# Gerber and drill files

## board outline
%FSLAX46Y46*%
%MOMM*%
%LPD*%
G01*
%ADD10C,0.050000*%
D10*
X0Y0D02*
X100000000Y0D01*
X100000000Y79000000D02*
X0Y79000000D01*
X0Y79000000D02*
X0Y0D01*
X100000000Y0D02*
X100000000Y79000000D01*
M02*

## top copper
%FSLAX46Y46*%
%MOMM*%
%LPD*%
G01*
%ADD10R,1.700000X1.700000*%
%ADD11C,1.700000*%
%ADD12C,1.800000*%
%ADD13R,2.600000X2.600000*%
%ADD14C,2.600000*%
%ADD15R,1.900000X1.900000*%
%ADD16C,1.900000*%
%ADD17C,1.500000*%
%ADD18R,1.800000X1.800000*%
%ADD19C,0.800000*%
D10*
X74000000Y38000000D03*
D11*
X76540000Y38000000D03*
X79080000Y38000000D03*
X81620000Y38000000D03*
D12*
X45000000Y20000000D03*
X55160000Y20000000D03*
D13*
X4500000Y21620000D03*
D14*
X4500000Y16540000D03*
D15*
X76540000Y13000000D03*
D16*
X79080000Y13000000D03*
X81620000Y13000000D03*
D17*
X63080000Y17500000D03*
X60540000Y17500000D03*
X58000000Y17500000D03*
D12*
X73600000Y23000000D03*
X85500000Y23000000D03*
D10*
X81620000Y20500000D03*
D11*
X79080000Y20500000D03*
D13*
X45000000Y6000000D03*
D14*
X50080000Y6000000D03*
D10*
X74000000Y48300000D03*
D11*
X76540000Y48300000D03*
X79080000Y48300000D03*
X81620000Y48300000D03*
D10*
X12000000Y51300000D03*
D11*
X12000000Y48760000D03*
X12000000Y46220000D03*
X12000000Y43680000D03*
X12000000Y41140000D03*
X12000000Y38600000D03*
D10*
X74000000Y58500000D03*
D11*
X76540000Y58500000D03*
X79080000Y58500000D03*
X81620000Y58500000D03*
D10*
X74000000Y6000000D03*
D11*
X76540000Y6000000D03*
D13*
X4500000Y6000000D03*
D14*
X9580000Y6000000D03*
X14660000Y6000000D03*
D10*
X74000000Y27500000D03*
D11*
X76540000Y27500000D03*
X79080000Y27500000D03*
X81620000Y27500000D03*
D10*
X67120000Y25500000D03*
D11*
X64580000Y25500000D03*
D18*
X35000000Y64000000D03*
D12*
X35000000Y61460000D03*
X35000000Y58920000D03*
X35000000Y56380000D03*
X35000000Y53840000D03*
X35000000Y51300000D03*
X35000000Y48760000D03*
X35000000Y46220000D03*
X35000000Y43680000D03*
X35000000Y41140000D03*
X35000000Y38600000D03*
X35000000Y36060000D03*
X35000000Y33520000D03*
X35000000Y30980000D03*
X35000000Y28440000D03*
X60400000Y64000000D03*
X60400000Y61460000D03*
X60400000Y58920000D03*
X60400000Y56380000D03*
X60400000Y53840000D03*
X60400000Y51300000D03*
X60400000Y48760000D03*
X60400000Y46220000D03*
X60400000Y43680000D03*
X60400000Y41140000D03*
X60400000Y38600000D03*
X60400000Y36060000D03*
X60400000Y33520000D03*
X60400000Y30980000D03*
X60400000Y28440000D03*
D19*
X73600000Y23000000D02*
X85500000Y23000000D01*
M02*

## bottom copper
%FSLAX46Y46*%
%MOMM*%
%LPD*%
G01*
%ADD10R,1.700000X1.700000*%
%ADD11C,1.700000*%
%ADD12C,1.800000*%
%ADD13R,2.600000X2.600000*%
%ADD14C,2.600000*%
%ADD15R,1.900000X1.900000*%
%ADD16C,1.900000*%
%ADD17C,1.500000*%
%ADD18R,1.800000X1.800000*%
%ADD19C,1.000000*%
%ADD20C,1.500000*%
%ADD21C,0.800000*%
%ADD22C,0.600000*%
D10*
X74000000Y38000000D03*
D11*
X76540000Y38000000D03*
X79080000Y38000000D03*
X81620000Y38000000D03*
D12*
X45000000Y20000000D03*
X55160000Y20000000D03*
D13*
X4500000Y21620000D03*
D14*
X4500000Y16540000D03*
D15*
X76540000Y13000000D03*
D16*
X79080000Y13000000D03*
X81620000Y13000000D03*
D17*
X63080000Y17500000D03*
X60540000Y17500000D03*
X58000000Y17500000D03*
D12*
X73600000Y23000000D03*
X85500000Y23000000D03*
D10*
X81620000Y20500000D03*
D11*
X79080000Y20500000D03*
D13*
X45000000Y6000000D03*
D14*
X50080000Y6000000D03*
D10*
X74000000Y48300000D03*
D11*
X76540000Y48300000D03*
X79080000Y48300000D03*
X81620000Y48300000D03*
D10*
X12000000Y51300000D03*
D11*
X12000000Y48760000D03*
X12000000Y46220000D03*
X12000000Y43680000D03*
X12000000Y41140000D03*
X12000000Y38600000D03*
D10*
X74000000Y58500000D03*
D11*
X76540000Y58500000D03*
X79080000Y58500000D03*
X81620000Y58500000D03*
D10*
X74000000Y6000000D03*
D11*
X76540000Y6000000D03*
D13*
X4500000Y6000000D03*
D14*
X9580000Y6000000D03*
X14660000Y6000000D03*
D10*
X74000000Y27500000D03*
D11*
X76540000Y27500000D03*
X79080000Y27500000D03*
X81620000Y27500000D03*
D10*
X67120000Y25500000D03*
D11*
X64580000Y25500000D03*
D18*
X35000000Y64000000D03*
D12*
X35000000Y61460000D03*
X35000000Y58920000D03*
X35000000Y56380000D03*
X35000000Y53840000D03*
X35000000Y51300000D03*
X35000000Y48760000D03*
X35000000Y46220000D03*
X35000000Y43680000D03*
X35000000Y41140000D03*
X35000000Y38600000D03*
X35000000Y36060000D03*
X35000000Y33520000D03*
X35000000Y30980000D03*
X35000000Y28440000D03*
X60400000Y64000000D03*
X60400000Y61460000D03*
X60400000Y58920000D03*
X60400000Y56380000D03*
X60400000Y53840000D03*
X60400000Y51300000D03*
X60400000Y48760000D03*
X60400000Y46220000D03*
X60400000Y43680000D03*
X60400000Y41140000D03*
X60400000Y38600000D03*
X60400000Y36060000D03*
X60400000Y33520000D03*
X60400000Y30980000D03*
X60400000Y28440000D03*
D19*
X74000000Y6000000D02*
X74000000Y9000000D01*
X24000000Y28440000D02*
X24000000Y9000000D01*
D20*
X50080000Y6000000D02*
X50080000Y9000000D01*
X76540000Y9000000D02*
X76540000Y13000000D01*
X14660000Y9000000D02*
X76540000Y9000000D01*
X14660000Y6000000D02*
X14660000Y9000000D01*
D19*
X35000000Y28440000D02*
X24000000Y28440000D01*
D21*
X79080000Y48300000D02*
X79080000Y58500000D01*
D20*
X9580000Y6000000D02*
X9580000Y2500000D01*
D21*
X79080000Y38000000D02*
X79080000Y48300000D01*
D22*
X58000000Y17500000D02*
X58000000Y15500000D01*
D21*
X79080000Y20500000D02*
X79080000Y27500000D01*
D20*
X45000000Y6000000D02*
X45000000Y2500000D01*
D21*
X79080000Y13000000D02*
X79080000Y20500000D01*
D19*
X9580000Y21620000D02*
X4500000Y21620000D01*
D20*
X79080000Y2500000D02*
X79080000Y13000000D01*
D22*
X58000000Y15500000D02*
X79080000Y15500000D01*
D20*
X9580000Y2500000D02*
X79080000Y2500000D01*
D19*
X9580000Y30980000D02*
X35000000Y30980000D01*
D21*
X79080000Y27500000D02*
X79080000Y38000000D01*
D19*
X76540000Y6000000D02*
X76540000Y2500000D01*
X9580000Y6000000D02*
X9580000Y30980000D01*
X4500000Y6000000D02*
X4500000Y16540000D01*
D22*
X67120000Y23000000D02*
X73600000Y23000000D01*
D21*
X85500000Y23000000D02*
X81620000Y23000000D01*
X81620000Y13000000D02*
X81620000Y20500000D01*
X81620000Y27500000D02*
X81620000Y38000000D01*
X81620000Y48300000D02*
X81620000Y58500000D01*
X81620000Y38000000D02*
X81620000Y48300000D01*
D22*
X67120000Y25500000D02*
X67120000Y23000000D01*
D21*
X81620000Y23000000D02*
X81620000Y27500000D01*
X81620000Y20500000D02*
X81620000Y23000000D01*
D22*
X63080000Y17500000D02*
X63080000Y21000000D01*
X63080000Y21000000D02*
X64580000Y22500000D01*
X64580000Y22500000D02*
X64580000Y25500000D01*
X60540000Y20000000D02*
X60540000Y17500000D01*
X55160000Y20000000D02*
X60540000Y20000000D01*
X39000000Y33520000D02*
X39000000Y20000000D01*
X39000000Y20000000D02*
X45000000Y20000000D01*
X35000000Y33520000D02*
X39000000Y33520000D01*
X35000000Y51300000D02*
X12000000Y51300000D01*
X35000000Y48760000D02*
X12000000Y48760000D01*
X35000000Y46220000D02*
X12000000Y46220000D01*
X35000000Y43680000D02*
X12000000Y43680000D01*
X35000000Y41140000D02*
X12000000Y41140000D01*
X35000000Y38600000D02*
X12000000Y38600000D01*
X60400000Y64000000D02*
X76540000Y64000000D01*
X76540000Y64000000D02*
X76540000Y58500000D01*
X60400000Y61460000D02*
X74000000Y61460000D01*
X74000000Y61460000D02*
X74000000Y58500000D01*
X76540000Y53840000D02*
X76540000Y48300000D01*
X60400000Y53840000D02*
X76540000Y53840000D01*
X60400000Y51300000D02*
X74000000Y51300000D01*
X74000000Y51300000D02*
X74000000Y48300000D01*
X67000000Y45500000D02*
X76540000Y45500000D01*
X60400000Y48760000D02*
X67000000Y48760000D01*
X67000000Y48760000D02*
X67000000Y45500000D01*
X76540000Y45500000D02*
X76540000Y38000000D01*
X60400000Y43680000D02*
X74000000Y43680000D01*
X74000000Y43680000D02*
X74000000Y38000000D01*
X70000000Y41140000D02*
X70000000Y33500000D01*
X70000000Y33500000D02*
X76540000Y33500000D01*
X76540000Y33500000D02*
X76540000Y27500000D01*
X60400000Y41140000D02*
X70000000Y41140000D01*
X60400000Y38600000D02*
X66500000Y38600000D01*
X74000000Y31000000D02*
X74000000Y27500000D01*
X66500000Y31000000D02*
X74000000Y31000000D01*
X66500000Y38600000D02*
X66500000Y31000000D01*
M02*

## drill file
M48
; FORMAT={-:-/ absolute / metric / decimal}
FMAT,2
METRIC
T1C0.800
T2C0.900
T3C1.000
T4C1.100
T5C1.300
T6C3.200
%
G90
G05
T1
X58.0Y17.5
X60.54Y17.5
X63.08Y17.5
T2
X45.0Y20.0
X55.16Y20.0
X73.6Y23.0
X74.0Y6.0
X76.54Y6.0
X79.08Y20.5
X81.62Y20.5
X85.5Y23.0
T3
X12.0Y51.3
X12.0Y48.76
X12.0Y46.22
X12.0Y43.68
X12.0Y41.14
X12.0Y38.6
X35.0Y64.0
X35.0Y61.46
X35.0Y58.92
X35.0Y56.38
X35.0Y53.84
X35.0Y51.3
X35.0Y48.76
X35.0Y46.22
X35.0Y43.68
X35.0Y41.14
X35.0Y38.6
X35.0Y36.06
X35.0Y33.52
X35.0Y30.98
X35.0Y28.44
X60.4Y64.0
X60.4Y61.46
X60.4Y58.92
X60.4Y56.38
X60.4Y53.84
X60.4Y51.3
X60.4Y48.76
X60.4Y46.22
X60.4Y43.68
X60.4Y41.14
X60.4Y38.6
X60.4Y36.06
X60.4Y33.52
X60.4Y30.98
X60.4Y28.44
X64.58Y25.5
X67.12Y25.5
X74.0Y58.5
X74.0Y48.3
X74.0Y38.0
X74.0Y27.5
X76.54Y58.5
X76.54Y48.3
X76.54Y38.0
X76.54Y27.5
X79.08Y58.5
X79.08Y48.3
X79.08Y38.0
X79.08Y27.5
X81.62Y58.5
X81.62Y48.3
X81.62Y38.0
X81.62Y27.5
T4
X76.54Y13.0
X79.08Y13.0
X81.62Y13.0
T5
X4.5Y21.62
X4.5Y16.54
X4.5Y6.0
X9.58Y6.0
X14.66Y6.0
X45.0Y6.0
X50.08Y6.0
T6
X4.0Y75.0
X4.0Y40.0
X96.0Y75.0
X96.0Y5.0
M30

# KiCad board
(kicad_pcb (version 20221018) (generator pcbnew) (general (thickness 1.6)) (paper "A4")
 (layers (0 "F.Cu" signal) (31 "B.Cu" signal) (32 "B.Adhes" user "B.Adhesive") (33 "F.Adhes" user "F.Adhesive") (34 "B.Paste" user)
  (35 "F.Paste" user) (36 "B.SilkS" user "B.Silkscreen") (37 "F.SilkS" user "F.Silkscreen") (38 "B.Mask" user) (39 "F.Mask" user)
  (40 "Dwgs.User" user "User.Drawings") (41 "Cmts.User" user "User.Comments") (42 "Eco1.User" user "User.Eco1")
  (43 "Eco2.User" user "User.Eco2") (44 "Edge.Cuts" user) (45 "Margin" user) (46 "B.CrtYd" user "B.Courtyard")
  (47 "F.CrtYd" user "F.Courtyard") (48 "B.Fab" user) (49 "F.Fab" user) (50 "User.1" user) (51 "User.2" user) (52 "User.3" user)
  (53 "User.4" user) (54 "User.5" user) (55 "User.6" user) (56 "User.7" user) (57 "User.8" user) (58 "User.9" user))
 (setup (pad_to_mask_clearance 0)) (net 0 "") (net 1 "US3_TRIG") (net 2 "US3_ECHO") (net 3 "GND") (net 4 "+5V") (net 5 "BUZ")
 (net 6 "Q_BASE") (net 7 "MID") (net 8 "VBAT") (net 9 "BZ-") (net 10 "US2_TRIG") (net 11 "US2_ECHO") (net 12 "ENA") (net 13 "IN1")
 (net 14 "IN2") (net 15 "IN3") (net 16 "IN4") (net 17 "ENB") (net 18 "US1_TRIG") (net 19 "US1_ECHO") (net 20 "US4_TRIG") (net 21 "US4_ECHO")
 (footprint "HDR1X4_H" (layer "F.Cu") (at 77.81 -38)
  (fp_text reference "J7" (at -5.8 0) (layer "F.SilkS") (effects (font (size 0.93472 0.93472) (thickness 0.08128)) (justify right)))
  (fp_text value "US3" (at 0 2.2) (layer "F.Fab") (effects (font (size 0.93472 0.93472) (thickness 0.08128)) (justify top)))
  (pad "1" thru_hole rect (at -3.81 0) (size 1.7 1.7) (drill 1) (layers "*.Cu" "*.Mask") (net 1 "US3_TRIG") (solder_mask_margin 0.1)
   (thermal_bridge_angle 0))
  (pad "2" thru_hole circle (at -1.27 0) (size 1.7 1.7) (drill 1) (layers "*.Cu" "*.Mask") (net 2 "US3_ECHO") (solder_mask_margin 0.1)
   (thermal_bridge_angle 0))
  (pad "3" thru_hole circle (at 1.27 0) (size 1.7 1.7) (drill 1) (layers "*.Cu" "*.Mask") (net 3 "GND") (solder_mask_margin 0.1)
   (thermal_bridge_angle 0))
  (pad "4" thru_hole circle (at 3.81 0) (size 1.7 1.7) (drill 1) (layers "*.Cu" "*.Mask") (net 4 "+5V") (solder_mask_margin 0.1)
   (thermal_bridge_angle 0)))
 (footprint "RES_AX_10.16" (layer "F.Cu") (at 50.08 -20)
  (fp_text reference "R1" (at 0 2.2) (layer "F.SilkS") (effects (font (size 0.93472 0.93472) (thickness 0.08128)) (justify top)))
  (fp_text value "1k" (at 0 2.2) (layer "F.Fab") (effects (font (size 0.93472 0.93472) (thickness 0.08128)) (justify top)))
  (pad "1" thru_hole circle (at -5.08 0) (size 1.8 1.8) (drill 0.9) (layers "*.Cu" "*.Mask") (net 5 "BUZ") (solder_mask_margin 0.1)
   (thermal_bridge_angle 0))
  (pad "2" thru_hole circle (at 5.08 0) (size 1.8 1.8) (drill 0.9) (layers "*.Cu" "*.Mask") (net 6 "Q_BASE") (solder_mask_margin 0.1)
   (thermal_bridge_angle 0)))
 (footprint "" (layer "F.Cu") (at 96 -75)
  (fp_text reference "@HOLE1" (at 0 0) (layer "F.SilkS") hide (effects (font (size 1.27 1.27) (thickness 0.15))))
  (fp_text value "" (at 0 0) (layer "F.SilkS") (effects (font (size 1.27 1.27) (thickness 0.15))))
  (pad "" np_thru_hole circle (at 0 0) (size 3.2 3.2) (drill 3.2) (layers "*.Cu" "*.Mask")))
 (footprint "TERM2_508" (layer "F.Cu") (at 4.5 -19.08 -90)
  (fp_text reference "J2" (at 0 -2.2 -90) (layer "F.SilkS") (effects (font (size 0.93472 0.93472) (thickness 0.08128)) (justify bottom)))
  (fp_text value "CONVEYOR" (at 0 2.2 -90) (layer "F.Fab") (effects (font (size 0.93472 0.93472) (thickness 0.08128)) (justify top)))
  (pad "1" thru_hole rect (at -2.54 0 270) (size 2.6 2.6) (drill 1.3) (layers "*.Cu" "*.Mask") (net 3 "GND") (solder_mask_margin 0.1)
   (thermal_bridge_angle 0))
  (pad "2" thru_hole circle (at 2.54 0 270) (size 2.6 2.6) (drill 1.3) (layers "*.Cu" "*.Mask") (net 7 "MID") (solder_mask_margin 0.1)
   (thermal_bridge_angle 0)))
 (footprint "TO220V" (layer "F.Cu") (at 79.08 -13)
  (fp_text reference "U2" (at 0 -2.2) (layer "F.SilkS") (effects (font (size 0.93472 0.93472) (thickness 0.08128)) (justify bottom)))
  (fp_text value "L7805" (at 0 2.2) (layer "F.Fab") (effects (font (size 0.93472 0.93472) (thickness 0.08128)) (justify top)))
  (pad "1" thru_hole rect (at -2.54 0) (size 1.9 1.9) (drill 1.1) (layers "*.Cu" "*.Mask") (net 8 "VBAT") (solder_mask_margin 0.1)
   (thermal_bridge_angle 0))
  (pad "2" thru_hole circle (at 0 0) (size 1.9 1.9) (drill 1.1) (layers "*.Cu" "*.Mask") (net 3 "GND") (solder_mask_margin 0.1)
   (thermal_bridge_angle 0))
  (pad "3" thru_hole circle (at 2.54 0) (size 1.9 1.9) (drill 1.1) (layers "*.Cu" "*.Mask") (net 4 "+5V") (solder_mask_margin 0.1)
   (thermal_bridge_angle 0)))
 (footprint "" (layer "F.Cu") (at 96 -5)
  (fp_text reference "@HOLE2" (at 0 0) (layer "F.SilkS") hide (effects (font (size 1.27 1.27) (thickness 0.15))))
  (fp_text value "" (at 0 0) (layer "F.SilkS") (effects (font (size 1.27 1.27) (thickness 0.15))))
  (pad "" np_thru_hole circle (at 0 0) (size 3.2 3.2) (drill 3.2) (layers "*.Cu" "*.Mask")))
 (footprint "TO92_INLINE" (layer "F.Cu") (at 60.54 -17.5 180)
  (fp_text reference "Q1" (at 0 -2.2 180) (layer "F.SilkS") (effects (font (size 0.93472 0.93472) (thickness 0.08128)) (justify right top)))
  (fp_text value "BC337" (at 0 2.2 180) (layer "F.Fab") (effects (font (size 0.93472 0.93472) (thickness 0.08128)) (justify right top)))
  (pad "1" thru_hole circle (at -2.54 0 180) (size 1.5 1.5) (drill 0.8) (layers "*.Cu" "*.Mask") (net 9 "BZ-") (solder_mask_margin 0.1)
   (thermal_bridge_angle 0))
  (pad "2" thru_hole circle (at 0 0 180) (size 1.5 1.5) (drill 0.8) (layers "*.Cu" "*.Mask") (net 6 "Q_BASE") (solder_mask_margin 0.1)
   (thermal_bridge_angle 0))
  (pad "3" thru_hole circle (at 2.54 0 180) (size 1.5 1.5) (drill 0.8) (layers "*.Cu" "*.Mask") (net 3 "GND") (solder_mask_margin 0.1)
   (thermal_bridge_angle 0)))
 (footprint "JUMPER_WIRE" (layer "F.Cu") (at 73.6 -23)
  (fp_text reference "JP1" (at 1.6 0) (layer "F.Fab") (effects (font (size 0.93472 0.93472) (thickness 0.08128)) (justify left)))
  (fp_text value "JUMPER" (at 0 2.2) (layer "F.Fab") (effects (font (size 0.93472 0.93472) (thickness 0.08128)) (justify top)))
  (pad "1" thru_hole circle (at 0 0) (size 1.8 1.8) (drill 0.9) (layers "*.Cu" "*.Mask") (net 4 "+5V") (solder_mask_margin 0.1)
   (thermal_bridge_angle 0))
  (pad "2" thru_hole circle (at 11.9 0) (size 1.8 1.8) (drill 0.9) (layers "*.Cu" "*.Mask") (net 4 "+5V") (solder_mask_margin 0.1)
   (thermal_bridge_angle 0)))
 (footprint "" (layer "F.Cu") (at 4 -75)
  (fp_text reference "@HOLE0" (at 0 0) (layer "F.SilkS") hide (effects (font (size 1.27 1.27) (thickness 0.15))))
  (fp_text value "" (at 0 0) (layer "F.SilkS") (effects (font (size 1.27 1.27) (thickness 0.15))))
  (pad "" np_thru_hole circle (at 0 0) (size 3.2 3.2) (drill 3.2) (layers "*.Cu" "*.Mask")))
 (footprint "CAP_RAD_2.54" (layer "F.Cu") (at 80.35 -20.5 180)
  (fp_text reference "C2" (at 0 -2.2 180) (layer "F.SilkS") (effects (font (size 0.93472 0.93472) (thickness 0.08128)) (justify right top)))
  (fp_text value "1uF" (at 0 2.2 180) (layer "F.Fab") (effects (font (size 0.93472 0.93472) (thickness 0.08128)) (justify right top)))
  (pad "1" thru_hole rect (at -1.27 0 180) (size 1.7 1.7) (drill 0.9) (layers "*.Cu" "*.Mask") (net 4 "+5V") (solder_mask_margin 0.1)
   (thermal_bridge_angle 0))
  (pad "2" thru_hole circle (at 1.27 0 180) (size 1.7 1.7) (drill 0.9) (layers "*.Cu" "*.Mask") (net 3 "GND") (solder_mask_margin 0.1)
   (thermal_bridge_angle 0)))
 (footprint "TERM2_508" (layer "F.Cu") (at 47.54 -6)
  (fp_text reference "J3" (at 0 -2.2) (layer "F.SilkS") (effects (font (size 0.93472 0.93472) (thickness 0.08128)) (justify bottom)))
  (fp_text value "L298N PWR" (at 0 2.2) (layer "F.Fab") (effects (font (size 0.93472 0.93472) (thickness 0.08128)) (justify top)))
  (pad "1" thru_hole rect (at -2.54 0) (size 2.6 2.6) (drill 1.3) (layers "*.Cu" "*.Mask") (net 3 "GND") (solder_mask_margin 0.1)
   (thermal_bridge_angle 0))
  (pad "2" thru_hole circle (at 2.54 0) (size 2.6 2.6) (drill 1.3) (layers "*.Cu" "*.Mask") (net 8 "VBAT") (solder_mask_margin 0.1)
   (thermal_bridge_angle 0)))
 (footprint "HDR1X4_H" (layer "F.Cu") (at 77.81 -48.3)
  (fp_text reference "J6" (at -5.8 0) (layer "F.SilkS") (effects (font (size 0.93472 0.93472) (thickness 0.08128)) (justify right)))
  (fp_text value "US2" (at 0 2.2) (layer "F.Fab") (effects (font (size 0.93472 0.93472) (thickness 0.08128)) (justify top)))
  (pad "1" thru_hole rect (at -3.81 0) (size 1.7 1.7) (drill 1) (layers "*.Cu" "*.Mask") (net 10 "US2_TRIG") (solder_mask_margin 0.1)
   (thermal_bridge_angle 0))
  (pad "2" thru_hole circle (at -1.27 0) (size 1.7 1.7) (drill 1) (layers "*.Cu" "*.Mask") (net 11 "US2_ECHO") (solder_mask_margin 0.1)
   (thermal_bridge_angle 0))
  (pad "3" thru_hole circle (at 1.27 0) (size 1.7 1.7) (drill 1) (layers "*.Cu" "*.Mask") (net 3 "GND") (solder_mask_margin 0.1)
   (thermal_bridge_angle 0))
  (pad "4" thru_hole circle (at 3.81 0) (size 1.7 1.7) (drill 1) (layers "*.Cu" "*.Mask") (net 4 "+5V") (solder_mask_margin 0.1)
   (thermal_bridge_angle 0)))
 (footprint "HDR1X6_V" (layer "F.Cu") (at 12 -44.95)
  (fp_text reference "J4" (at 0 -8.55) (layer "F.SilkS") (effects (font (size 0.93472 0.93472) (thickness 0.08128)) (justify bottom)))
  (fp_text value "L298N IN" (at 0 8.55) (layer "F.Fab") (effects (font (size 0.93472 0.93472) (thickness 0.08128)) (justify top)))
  (pad "1" thru_hole rect (at 0 -6.35) (size 1.7 1.7) (drill 1) (layers "*.Cu" "*.Mask") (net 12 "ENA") (solder_mask_margin 0.1)
   (thermal_bridge_angle 0))
  (pad "2" thru_hole circle (at 0 -3.81) (size 1.7 1.7) (drill 1) (layers "*.Cu" "*.Mask") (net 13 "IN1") (solder_mask_margin 0.1)
   (thermal_bridge_angle 0))
  (pad "3" thru_hole circle (at 0 -1.27) (size 1.7 1.7) (drill 1) (layers "*.Cu" "*.Mask") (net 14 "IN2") (solder_mask_margin 0.1)
   (thermal_bridge_angle 0))
  (pad "4" thru_hole circle (at 0 1.27) (size 1.7 1.7) (drill 1) (layers "*.Cu" "*.Mask") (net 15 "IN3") (solder_mask_margin 0.1)
   (thermal_bridge_angle 0))
  (pad "5" thru_hole circle (at 0 3.81) (size 1.7 1.7) (drill 1) (layers "*.Cu" "*.Mask") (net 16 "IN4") (solder_mask_margin 0.1)
   (thermal_bridge_angle 0))
  (pad "6" thru_hole circle (at 0 6.35) (size 1.7 1.7) (drill 1) (layers "*.Cu" "*.Mask") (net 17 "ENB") (solder_mask_margin 0.1)
   (thermal_bridge_angle 0)))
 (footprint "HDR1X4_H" (layer "F.Cu") (at 77.81 -58.5)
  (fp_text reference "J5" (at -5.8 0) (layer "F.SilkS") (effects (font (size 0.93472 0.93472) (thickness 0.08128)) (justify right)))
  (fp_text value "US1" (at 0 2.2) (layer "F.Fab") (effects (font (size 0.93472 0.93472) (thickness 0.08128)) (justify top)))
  (pad "1" thru_hole rect (at -3.81 0) (size 1.7 1.7) (drill 1) (layers "*.Cu" "*.Mask") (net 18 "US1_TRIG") (solder_mask_margin 0.1)
   (thermal_bridge_angle 0))
  (pad "2" thru_hole circle (at -1.27 0) (size 1.7 1.7) (drill 1) (layers "*.Cu" "*.Mask") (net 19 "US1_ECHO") (solder_mask_margin 0.1)
   (thermal_bridge_angle 0))
  (pad "3" thru_hole circle (at 1.27 0) (size 1.7 1.7) (drill 1) (layers "*.Cu" "*.Mask") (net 3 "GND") (solder_mask_margin 0.1)
   (thermal_bridge_angle 0))
  (pad "4" thru_hole circle (at 3.81 0) (size 1.7 1.7) (drill 1) (layers "*.Cu" "*.Mask") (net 4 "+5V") (solder_mask_margin 0.1)
   (thermal_bridge_angle 0)))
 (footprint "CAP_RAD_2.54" (layer "F.Cu") (at 75.27 -6)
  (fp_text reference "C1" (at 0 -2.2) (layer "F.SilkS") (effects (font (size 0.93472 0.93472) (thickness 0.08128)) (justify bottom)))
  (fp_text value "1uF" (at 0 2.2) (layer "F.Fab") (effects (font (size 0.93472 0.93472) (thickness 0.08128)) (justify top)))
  (pad "1" thru_hole rect (at -1.27 0) (size 1.7 1.7) (drill 0.9) (layers "*.Cu" "*.Mask") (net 8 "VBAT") (solder_mask_margin 0.1)
   (thermal_bridge_angle 0))
  (pad "2" thru_hole circle (at 1.27 0) (size 1.7 1.7) (drill 0.9) (layers "*.Cu" "*.Mask") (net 3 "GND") (solder_mask_margin 0.1)
   (thermal_bridge_angle 0)))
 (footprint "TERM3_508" (layer "F.Cu") (at 9.58 -6)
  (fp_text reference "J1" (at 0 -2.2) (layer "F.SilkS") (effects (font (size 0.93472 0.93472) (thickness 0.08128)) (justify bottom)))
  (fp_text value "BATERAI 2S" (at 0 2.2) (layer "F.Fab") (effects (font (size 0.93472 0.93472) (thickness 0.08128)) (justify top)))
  (pad "1" thru_hole rect (at -5.08 0) (size 2.6 2.6) (drill 1.3) (layers "*.Cu" "*.Mask") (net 7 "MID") (solder_mask_margin 0.1)
   (thermal_bridge_angle 0))
  (pad "2" thru_hole circle (at 0 0) (size 2.6 2.6) (drill 1.3) (layers "*.Cu" "*.Mask") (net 3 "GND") (solder_mask_margin 0.1)
   (thermal_bridge_angle 0))
  (pad "3" thru_hole circle (at 5.08 0) (size 2.6 2.6) (drill 1.3) (layers "*.Cu" "*.Mask") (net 8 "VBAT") (solder_mask_margin 0.1)
   (thermal_bridge_angle 0)))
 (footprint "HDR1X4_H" (layer "F.Cu") (at 77.81 -27.5)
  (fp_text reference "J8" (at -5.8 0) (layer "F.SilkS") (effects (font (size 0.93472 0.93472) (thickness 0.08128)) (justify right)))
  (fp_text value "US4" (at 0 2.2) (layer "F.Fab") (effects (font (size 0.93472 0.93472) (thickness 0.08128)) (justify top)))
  (pad "1" thru_hole rect (at -3.81 0) (size 1.7 1.7) (drill 1) (layers "*.Cu" "*.Mask") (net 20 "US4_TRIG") (solder_mask_margin 0.1)
   (thermal_bridge_angle 0))
  (pad "2" thru_hole circle (at -1.27 0) (size 1.7 1.7) (drill 1) (layers "*.Cu" "*.Mask") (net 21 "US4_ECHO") (solder_mask_margin 0.1)
   (thermal_bridge_angle 0))
  (pad "3" thru_hole circle (at 1.27 0) (size 1.7 1.7) (drill 1) (layers "*.Cu" "*.Mask") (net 3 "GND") (solder_mask_margin 0.1)
   (thermal_bridge_angle 0))
  (pad "4" thru_hole circle (at 3.81 0) (size 1.7 1.7) (drill 1) (layers "*.Cu" "*.Mask") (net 4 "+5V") (solder_mask_margin 0.1)
   (thermal_bridge_angle 0)))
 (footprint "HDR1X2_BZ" (layer "F.Cu") (at 65.85 -25.5)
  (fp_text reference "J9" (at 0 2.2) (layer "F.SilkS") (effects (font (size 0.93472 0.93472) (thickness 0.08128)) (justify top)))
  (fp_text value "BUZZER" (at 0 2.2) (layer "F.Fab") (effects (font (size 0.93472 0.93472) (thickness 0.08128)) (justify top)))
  (pad "1" thru_hole rect (at 1.27 0) (size 1.7 1.7) (drill 1) (layers "*.Cu" "*.Mask") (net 4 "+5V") (solder_mask_margin 0.1)
   (thermal_bridge_angle 0))
  (pad "2" thru_hole circle (at -1.27 0) (size 1.7 1.7) (drill 1) (layers "*.Cu" "*.Mask") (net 9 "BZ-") (solder_mask_margin 0.1)
   (thermal_bridge_angle 0)))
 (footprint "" (layer "F.Cu") (at 4 -40)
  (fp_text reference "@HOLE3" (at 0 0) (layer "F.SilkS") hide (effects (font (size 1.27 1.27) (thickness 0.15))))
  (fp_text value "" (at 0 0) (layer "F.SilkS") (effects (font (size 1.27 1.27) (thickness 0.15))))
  (pad "" np_thru_hole circle (at 0 0) (size 3.2 3.2) (drill 3.2) (layers "*.Cu" "*.Mask")))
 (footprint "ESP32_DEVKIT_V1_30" (layer "F.Cu") (at 47.7 -46.22)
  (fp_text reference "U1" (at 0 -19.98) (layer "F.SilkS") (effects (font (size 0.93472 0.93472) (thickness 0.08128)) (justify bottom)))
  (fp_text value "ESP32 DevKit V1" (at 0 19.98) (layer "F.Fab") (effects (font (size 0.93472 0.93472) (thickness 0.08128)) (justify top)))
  (pad "L1" thru_hole rect (at -12.7 -17.78) (size 1.8 1.8) (drill 1) (layers "*.Cu" "*.Mask") (solder_mask_margin 0.1)
   (thermal_bridge_angle 0))
  (pad "L2" thru_hole circle (at -12.7 -15.24) (size 1.8 1.8) (drill 1) (layers "*.Cu" "*.Mask") (solder_mask_margin 0.1)
   (thermal_bridge_angle 0))
  (pad "L3" thru_hole circle (at -12.7 -12.7) (size 1.8 1.8) (drill 1) (layers "*.Cu" "*.Mask") (solder_mask_margin 0.1)
   (thermal_bridge_angle 0))
  (pad "L4" thru_hole circle (at -12.7 -10.16) (size 1.8 1.8) (drill 1) (layers "*.Cu" "*.Mask") (solder_mask_margin 0.1)
   (thermal_bridge_angle 0))
  (pad "L5" thru_hole circle (at -12.7 -7.62) (size 1.8 1.8) (drill 1) (layers "*.Cu" "*.Mask") (solder_mask_margin 0.1)
   (thermal_bridge_angle 0))
  (pad "L6" thru_hole circle (at -12.7 -5.08) (size 1.8 1.8) (drill 1) (layers "*.Cu" "*.Mask") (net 12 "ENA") (solder_mask_margin 0.1)
   (thermal_bridge_angle 0))
  (pad "L7" thru_hole circle (at -12.7 -2.54) (size 1.8 1.8) (drill 1) (layers "*.Cu" "*.Mask") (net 13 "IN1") (solder_mask_margin 0.1)
   (thermal_bridge_angle 0))
  (pad "L8" thru_hole circle (at -12.7 0) (size 1.8 1.8) (drill 1) (layers "*.Cu" "*.Mask") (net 14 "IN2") (solder_mask_margin 0.1)
   (thermal_bridge_angle 0))
  (pad "L9" thru_hole circle (at -12.7 2.54) (size 1.8 1.8) (drill 1) (layers "*.Cu" "*.Mask") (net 15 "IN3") (solder_mask_margin 0.1)
   (thermal_bridge_angle 0))
  (pad "L10" thru_hole circle (at -12.7 5.08) (size 1.8 1.8) (drill 1) (layers "*.Cu" "*.Mask") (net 16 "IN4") (solder_mask_margin 0.1)
   (thermal_bridge_angle 0))
  (pad "L11" thru_hole circle (at -12.7 7.62) (size 1.8 1.8) (drill 1) (layers "*.Cu" "*.Mask") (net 17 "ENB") (solder_mask_margin 0.1)
   (thermal_bridge_angle 0))
  (pad "L12" thru_hole circle (at -12.7 10.16) (size 1.8 1.8) (drill 1) (layers "*.Cu" "*.Mask") (solder_mask_margin 0.1)
   (thermal_bridge_angle 0))
  (pad "L13" thru_hole circle (at -12.7 12.7) (size 1.8 1.8) (drill 1) (layers "*.Cu" "*.Mask") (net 5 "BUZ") (solder_mask_margin 0.1)
   (thermal_bridge_angle 0))
  (pad "L14" thru_hole circle (at -12.7 15.24) (size 1.8 1.8) (drill 1) (layers "*.Cu" "*.Mask") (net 3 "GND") (solder_mask_margin 0.1)
   (thermal_bridge_angle 0))
  (pad "L15" thru_hole circle (at -12.7 17.78) (size 1.8 1.8) (drill 1) (layers "*.Cu" "*.Mask") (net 8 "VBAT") (solder_mask_margin 0.1)
   (thermal_bridge_angle 0))
  (pad "R1" thru_hole circle (at 12.7 -17.78) (size 1.8 1.8) (drill 1) (layers "*.Cu" "*.Mask") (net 19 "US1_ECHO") (solder_mask_margin 0.1)
   (thermal_bridge_angle 0))
  (pad "R2" thru_hole circle (at 12.7 -15.24) (size 1.8 1.8) (drill 1) (layers "*.Cu" "*.Mask") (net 18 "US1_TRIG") (solder_mask_margin 0.1)
   (thermal_bridge_angle 0))
  (pad "R3" thru_hole circle (at 12.7 -12.7) (size 1.8 1.8) (drill 1) (layers "*.Cu" "*.Mask") (solder_mask_margin 0.1)
   (thermal_bridge_angle 0))
  (pad "R4" thru_hole circle (at 12.7 -10.16) (size 1.8 1.8) (drill 1) (layers "*.Cu" "*.Mask") (solder_mask_margin 0.1)
   (thermal_bridge_angle 0))
  (pad "R5" thru_hole circle (at 12.7 -7.62) (size 1.8 1.8) (drill 1) (layers "*.Cu" "*.Mask") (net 11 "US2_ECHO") (solder_mask_margin 0.1)
   (thermal_bridge_angle 0))
  (pad "R6" thru_hole circle (at 12.7 -5.08) (size 1.8 1.8) (drill 1) (layers "*.Cu" "*.Mask") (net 10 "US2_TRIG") (solder_mask_margin 0.1)
   (thermal_bridge_angle 0))
  (pad "R7" thru_hole circle (at 12.7 -2.54) (size 1.8 1.8) (drill 1) (layers "*.Cu" "*.Mask") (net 2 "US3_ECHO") (solder_mask_margin 0.1)
   (thermal_bridge_angle 0))
  (pad "R8" thru_hole circle (at 12.7 0) (size 1.8 1.8) (drill 1) (layers "*.Cu" "*.Mask") (solder_mask_margin 0.1) (thermal_bridge_angle 0))
  (pad "R9" thru_hole circle (at 12.7 2.54) (size 1.8 1.8) (drill 1) (layers "*.Cu" "*.Mask") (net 1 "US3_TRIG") (solder_mask_margin 0.1)
   (thermal_bridge_angle 0))
  (pad "R10" thru_hole circle (at 12.7 5.08) (size 1.8 1.8) (drill 1) (layers "*.Cu" "*.Mask") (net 21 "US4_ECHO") (solder_mask_margin 0.1)
   (thermal_bridge_angle 0))
  (pad "R11" thru_hole circle (at 12.7 7.62) (size 1.8 1.8) (drill 1) (layers "*.Cu" "*.Mask") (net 20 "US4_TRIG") (solder_mask_margin 0.1)
   (thermal_bridge_angle 0))
  (pad "R12" thru_hole circle (at 12.7 10.16) (size 1.8 1.8) (drill 1) (layers "*.Cu" "*.Mask") (solder_mask_margin 0.1)
   (thermal_bridge_angle 0))
  (pad "R13" thru_hole circle (at 12.7 12.7) (size 1.8 1.8) (drill 1) (layers "*.Cu" "*.Mask") (solder_mask_margin 0.1)
   (thermal_bridge_angle 0))
  (pad "R14" thru_hole circle (at 12.7 15.24) (size 1.8 1.8) (drill 1) (layers "*.Cu" "*.Mask") (solder_mask_margin 0.1)
   (thermal_bridge_angle 0))
  (pad "R15" thru_hole circle (at 12.7 17.78) (size 1.8 1.8) (drill 1) (layers "*.Cu" "*.Mask") (solder_mask_margin 0.1)
   (thermal_bridge_angle 0)))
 (gr_line (start 0 0) (end 100 0) (stroke (width 0.05) (type solid)) (layer "Edge.Cuts"))
 (gr_line (start 100 -79) (end 0 -79) (stroke (width 0.05) (type solid)) (layer "Edge.Cuts"))
 (gr_line (start 0 -79) (end 0 0) (stroke (width 0.05) (type solid)) (layer "Edge.Cuts"))
 (gr_line (start 100 0) (end 100 -79) (stroke (width 0.05) (type solid)) (layer "Edge.Cuts"))
 (segment (start 74 -6) (end 74 -9) (width 1) (layer "B.Cu") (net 8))
 (segment (start 24 -28.44) (end 24 -9) (width 1) (layer "B.Cu") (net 8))
 (segment (start 50.08 -6) (end 50.08 -9) (width 1.5) (layer "B.Cu") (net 8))
 (segment (start 76.54 -9) (end 76.54 -13) (width 1.5) (layer "B.Cu") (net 8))
 (segment (start 14.66 -9) (end 76.54 -9) (width 1.5) (layer "B.Cu") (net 8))
 (segment (start 14.66 -6) (end 14.66 -9) (width 1.5) (layer "B.Cu") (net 8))
 (segment (start 35 -28.44) (end 24 -28.44) (width 1) (layer "B.Cu") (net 8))
 (segment (start 79.08 -48.3) (end 79.08 -58.5) (width 0.8) (layer "B.Cu") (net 3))
 (segment (start 9.58 -6) (end 9.58 -2.5) (width 1.5) (layer "B.Cu") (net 3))
 (segment (start 79.08 -38) (end 79.08 -48.3) (width 0.8) (layer "B.Cu") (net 3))
 (segment (start 58 -17.5) (end 58 -15.5) (width 0.6) (layer "B.Cu") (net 3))
 (segment (start 79.08 -20.5) (end 79.08 -27.5) (width 0.8) (layer "B.Cu") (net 3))
 (segment (start 45 -6) (end 45 -2.5) (width 1.5) (layer "B.Cu") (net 3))
 (segment (start 79.08 -13) (end 79.08 -20.5) (width 0.8) (layer "B.Cu") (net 3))
 (segment (start 9.58 -21.62) (end 4.5 -21.62) (width 1) (layer "B.Cu") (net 3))
 (segment (start 79.08 -2.5) (end 79.08 -13) (width 1.5) (layer "B.Cu") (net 3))
 (segment (start 58 -15.5) (end 79.08 -15.5) (width 0.6) (layer "B.Cu") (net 3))
 (segment (start 9.58 -2.5) (end 79.08 -2.5) (width 1.5) (layer "B.Cu") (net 3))
 (segment (start 9.58 -30.98) (end 35 -30.98) (width 1) (layer "B.Cu") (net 3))
 (segment (start 79.08 -27.5) (end 79.08 -38) (width 0.8) (layer "B.Cu") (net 3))
 (segment (start 76.54 -6) (end 76.54 -2.5) (width 1) (layer "B.Cu") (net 3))
 (segment (start 9.58 -6) (end 9.58 -30.98) (width 1) (layer "B.Cu") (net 3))
 (segment (start 4.5 -6) (end 4.5 -16.54) (width 1) (layer "B.Cu") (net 7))
 (segment (start 73.6 -23) (end 85.5 -23) (width 0.8) (layer "F.Cu") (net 4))
 (segment (start 67.12 -23) (end 73.6 -23) (width 0.6) (layer "B.Cu") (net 4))
 (segment (start 85.5 -23) (end 81.62 -23) (width 0.8) (layer "B.Cu") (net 4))
 (segment (start 81.62 -13) (end 81.62 -20.5) (width 0.8) (layer "B.Cu") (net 4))
 (segment (start 81.62 -27.5) (end 81.62 -38) (width 0.8) (layer "B.Cu") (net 4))
 (segment (start 81.62 -48.3) (end 81.62 -58.5) (width 0.8) (layer "B.Cu") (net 4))
 (segment (start 81.62 -38) (end 81.62 -48.3) (width 0.8) (layer "B.Cu") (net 4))
 (segment (start 67.12 -25.5) (end 67.12 -23) (width 0.6) (layer "B.Cu") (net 4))
 (segment (start 81.62 -23) (end 81.62 -27.5) (width 0.8) (layer "B.Cu") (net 4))
 (segment (start 81.62 -20.5) (end 81.62 -23) (width 0.8) (layer "B.Cu") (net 4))
 (segment (start 63.08 -17.5) (end 63.08 -21) (width 0.6) (layer "B.Cu") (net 9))
 (segment (start 63.08 -21) (end 64.58 -22.5) (width 0.6) (layer "B.Cu") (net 9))
 (segment (start 64.58 -22.5) (end 64.58 -25.5) (width 0.6) (layer "B.Cu") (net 9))
 (segment (start 60.54 -20) (end 60.54 -17.5) (width 0.6) (layer "B.Cu") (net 6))
 (segment (start 55.16 -20) (end 60.54 -20) (width 0.6) (layer "B.Cu") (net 6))
 (segment (start 39 -33.52) (end 39 -20) (width 0.6) (layer "B.Cu") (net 5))
 (segment (start 39 -20) (end 45 -20) (width 0.6) (layer "B.Cu") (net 5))
 (segment (start 35 -33.52) (end 39 -33.52) (width 0.6) (layer "B.Cu") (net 5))
 (segment (start 35 -51.3) (end 12 -51.3) (width 0.6) (layer "B.Cu") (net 12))
 (segment (start 35 -48.76) (end 12 -48.76) (width 0.6) (layer "B.Cu") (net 13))
 (segment (start 35 -46.22) (end 12 -46.22) (width 0.6) (layer "B.Cu") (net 14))
 (segment (start 35 -43.68) (end 12 -43.68) (width 0.6) (layer "B.Cu") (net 15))
 (segment (start 35 -41.14) (end 12 -41.14) (width 0.6) (layer "B.Cu") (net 16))
 (segment (start 35 -38.6) (end 12 -38.6) (width 0.6) (layer "B.Cu") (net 17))
 (segment (start 60.4 -64) (end 76.54 -64) (width 0.6) (layer "B.Cu") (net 19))
 (segment (start 76.54 -64) (end 76.54 -58.5) (width 0.6) (layer "B.Cu") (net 19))
 (segment (start 60.4 -61.46) (end 74 -61.46) (width 0.6) (layer "B.Cu") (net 18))
 (segment (start 74 -61.46) (end 74 -58.5) (width 0.6) (layer "B.Cu") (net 18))
 (segment (start 76.54 -53.84) (end 76.54 -48.3) (width 0.6) (layer "B.Cu") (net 11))
 (segment (start 60.4 -53.84) (end 76.54 -53.84) (width 0.6) (layer "B.Cu") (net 11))
 (segment (start 60.4 -51.3) (end 74 -51.3) (width 0.6) (layer "B.Cu") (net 10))
 (segment (start 74 -51.3) (end 74 -48.3) (width 0.6) (layer "B.Cu") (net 10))
 (segment (start 67 -45.5) (end 76.54 -45.5) (width 0.6) (layer "B.Cu") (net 2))
 (segment (start 60.4 -48.76) (end 67 -48.76) (width 0.6) (layer "B.Cu") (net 2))
 (segment (start 67 -48.76) (end 67 -45.5) (width 0.6) (layer "B.Cu") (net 2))
 (segment (start 76.54 -45.5) (end 76.54 -38) (width 0.6) (layer "B.Cu") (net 2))
 (segment (start 60.4 -43.68) (end 74 -43.68) (width 0.6) (layer "B.Cu") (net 1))
 (segment (start 74 -43.68) (end 74 -38) (width 0.6) (layer "B.Cu") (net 1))
 (segment (start 70 -41.14) (end 70 -33.5) (width 0.6) (layer "B.Cu") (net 21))
 (segment (start 70 -33.5) (end 76.54 -33.5) (width 0.6) (layer "B.Cu") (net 21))
 (segment (start 76.54 -33.5) (end 76.54 -27.5) (width 0.6) (layer "B.Cu") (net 21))
 (segment (start 60.4 -41.14) (end 70 -41.14) (width 0.6) (layer "B.Cu") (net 21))
 (segment (start 60.4 -38.6) (end 66.5 -38.6) (width 0.6) (layer "B.Cu") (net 20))
 (segment (start 74 -31) (end 74 -27.5) (width 0.6) (layer "B.Cu") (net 20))
 (segment (start 66.5 -31) (end 74 -31) (width 0.6) (layer "B.Cu") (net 20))
 (segment (start 66.5 -38.6) (end 66.5 -31) (width 0.6) (layer "B.Cu") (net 20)))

